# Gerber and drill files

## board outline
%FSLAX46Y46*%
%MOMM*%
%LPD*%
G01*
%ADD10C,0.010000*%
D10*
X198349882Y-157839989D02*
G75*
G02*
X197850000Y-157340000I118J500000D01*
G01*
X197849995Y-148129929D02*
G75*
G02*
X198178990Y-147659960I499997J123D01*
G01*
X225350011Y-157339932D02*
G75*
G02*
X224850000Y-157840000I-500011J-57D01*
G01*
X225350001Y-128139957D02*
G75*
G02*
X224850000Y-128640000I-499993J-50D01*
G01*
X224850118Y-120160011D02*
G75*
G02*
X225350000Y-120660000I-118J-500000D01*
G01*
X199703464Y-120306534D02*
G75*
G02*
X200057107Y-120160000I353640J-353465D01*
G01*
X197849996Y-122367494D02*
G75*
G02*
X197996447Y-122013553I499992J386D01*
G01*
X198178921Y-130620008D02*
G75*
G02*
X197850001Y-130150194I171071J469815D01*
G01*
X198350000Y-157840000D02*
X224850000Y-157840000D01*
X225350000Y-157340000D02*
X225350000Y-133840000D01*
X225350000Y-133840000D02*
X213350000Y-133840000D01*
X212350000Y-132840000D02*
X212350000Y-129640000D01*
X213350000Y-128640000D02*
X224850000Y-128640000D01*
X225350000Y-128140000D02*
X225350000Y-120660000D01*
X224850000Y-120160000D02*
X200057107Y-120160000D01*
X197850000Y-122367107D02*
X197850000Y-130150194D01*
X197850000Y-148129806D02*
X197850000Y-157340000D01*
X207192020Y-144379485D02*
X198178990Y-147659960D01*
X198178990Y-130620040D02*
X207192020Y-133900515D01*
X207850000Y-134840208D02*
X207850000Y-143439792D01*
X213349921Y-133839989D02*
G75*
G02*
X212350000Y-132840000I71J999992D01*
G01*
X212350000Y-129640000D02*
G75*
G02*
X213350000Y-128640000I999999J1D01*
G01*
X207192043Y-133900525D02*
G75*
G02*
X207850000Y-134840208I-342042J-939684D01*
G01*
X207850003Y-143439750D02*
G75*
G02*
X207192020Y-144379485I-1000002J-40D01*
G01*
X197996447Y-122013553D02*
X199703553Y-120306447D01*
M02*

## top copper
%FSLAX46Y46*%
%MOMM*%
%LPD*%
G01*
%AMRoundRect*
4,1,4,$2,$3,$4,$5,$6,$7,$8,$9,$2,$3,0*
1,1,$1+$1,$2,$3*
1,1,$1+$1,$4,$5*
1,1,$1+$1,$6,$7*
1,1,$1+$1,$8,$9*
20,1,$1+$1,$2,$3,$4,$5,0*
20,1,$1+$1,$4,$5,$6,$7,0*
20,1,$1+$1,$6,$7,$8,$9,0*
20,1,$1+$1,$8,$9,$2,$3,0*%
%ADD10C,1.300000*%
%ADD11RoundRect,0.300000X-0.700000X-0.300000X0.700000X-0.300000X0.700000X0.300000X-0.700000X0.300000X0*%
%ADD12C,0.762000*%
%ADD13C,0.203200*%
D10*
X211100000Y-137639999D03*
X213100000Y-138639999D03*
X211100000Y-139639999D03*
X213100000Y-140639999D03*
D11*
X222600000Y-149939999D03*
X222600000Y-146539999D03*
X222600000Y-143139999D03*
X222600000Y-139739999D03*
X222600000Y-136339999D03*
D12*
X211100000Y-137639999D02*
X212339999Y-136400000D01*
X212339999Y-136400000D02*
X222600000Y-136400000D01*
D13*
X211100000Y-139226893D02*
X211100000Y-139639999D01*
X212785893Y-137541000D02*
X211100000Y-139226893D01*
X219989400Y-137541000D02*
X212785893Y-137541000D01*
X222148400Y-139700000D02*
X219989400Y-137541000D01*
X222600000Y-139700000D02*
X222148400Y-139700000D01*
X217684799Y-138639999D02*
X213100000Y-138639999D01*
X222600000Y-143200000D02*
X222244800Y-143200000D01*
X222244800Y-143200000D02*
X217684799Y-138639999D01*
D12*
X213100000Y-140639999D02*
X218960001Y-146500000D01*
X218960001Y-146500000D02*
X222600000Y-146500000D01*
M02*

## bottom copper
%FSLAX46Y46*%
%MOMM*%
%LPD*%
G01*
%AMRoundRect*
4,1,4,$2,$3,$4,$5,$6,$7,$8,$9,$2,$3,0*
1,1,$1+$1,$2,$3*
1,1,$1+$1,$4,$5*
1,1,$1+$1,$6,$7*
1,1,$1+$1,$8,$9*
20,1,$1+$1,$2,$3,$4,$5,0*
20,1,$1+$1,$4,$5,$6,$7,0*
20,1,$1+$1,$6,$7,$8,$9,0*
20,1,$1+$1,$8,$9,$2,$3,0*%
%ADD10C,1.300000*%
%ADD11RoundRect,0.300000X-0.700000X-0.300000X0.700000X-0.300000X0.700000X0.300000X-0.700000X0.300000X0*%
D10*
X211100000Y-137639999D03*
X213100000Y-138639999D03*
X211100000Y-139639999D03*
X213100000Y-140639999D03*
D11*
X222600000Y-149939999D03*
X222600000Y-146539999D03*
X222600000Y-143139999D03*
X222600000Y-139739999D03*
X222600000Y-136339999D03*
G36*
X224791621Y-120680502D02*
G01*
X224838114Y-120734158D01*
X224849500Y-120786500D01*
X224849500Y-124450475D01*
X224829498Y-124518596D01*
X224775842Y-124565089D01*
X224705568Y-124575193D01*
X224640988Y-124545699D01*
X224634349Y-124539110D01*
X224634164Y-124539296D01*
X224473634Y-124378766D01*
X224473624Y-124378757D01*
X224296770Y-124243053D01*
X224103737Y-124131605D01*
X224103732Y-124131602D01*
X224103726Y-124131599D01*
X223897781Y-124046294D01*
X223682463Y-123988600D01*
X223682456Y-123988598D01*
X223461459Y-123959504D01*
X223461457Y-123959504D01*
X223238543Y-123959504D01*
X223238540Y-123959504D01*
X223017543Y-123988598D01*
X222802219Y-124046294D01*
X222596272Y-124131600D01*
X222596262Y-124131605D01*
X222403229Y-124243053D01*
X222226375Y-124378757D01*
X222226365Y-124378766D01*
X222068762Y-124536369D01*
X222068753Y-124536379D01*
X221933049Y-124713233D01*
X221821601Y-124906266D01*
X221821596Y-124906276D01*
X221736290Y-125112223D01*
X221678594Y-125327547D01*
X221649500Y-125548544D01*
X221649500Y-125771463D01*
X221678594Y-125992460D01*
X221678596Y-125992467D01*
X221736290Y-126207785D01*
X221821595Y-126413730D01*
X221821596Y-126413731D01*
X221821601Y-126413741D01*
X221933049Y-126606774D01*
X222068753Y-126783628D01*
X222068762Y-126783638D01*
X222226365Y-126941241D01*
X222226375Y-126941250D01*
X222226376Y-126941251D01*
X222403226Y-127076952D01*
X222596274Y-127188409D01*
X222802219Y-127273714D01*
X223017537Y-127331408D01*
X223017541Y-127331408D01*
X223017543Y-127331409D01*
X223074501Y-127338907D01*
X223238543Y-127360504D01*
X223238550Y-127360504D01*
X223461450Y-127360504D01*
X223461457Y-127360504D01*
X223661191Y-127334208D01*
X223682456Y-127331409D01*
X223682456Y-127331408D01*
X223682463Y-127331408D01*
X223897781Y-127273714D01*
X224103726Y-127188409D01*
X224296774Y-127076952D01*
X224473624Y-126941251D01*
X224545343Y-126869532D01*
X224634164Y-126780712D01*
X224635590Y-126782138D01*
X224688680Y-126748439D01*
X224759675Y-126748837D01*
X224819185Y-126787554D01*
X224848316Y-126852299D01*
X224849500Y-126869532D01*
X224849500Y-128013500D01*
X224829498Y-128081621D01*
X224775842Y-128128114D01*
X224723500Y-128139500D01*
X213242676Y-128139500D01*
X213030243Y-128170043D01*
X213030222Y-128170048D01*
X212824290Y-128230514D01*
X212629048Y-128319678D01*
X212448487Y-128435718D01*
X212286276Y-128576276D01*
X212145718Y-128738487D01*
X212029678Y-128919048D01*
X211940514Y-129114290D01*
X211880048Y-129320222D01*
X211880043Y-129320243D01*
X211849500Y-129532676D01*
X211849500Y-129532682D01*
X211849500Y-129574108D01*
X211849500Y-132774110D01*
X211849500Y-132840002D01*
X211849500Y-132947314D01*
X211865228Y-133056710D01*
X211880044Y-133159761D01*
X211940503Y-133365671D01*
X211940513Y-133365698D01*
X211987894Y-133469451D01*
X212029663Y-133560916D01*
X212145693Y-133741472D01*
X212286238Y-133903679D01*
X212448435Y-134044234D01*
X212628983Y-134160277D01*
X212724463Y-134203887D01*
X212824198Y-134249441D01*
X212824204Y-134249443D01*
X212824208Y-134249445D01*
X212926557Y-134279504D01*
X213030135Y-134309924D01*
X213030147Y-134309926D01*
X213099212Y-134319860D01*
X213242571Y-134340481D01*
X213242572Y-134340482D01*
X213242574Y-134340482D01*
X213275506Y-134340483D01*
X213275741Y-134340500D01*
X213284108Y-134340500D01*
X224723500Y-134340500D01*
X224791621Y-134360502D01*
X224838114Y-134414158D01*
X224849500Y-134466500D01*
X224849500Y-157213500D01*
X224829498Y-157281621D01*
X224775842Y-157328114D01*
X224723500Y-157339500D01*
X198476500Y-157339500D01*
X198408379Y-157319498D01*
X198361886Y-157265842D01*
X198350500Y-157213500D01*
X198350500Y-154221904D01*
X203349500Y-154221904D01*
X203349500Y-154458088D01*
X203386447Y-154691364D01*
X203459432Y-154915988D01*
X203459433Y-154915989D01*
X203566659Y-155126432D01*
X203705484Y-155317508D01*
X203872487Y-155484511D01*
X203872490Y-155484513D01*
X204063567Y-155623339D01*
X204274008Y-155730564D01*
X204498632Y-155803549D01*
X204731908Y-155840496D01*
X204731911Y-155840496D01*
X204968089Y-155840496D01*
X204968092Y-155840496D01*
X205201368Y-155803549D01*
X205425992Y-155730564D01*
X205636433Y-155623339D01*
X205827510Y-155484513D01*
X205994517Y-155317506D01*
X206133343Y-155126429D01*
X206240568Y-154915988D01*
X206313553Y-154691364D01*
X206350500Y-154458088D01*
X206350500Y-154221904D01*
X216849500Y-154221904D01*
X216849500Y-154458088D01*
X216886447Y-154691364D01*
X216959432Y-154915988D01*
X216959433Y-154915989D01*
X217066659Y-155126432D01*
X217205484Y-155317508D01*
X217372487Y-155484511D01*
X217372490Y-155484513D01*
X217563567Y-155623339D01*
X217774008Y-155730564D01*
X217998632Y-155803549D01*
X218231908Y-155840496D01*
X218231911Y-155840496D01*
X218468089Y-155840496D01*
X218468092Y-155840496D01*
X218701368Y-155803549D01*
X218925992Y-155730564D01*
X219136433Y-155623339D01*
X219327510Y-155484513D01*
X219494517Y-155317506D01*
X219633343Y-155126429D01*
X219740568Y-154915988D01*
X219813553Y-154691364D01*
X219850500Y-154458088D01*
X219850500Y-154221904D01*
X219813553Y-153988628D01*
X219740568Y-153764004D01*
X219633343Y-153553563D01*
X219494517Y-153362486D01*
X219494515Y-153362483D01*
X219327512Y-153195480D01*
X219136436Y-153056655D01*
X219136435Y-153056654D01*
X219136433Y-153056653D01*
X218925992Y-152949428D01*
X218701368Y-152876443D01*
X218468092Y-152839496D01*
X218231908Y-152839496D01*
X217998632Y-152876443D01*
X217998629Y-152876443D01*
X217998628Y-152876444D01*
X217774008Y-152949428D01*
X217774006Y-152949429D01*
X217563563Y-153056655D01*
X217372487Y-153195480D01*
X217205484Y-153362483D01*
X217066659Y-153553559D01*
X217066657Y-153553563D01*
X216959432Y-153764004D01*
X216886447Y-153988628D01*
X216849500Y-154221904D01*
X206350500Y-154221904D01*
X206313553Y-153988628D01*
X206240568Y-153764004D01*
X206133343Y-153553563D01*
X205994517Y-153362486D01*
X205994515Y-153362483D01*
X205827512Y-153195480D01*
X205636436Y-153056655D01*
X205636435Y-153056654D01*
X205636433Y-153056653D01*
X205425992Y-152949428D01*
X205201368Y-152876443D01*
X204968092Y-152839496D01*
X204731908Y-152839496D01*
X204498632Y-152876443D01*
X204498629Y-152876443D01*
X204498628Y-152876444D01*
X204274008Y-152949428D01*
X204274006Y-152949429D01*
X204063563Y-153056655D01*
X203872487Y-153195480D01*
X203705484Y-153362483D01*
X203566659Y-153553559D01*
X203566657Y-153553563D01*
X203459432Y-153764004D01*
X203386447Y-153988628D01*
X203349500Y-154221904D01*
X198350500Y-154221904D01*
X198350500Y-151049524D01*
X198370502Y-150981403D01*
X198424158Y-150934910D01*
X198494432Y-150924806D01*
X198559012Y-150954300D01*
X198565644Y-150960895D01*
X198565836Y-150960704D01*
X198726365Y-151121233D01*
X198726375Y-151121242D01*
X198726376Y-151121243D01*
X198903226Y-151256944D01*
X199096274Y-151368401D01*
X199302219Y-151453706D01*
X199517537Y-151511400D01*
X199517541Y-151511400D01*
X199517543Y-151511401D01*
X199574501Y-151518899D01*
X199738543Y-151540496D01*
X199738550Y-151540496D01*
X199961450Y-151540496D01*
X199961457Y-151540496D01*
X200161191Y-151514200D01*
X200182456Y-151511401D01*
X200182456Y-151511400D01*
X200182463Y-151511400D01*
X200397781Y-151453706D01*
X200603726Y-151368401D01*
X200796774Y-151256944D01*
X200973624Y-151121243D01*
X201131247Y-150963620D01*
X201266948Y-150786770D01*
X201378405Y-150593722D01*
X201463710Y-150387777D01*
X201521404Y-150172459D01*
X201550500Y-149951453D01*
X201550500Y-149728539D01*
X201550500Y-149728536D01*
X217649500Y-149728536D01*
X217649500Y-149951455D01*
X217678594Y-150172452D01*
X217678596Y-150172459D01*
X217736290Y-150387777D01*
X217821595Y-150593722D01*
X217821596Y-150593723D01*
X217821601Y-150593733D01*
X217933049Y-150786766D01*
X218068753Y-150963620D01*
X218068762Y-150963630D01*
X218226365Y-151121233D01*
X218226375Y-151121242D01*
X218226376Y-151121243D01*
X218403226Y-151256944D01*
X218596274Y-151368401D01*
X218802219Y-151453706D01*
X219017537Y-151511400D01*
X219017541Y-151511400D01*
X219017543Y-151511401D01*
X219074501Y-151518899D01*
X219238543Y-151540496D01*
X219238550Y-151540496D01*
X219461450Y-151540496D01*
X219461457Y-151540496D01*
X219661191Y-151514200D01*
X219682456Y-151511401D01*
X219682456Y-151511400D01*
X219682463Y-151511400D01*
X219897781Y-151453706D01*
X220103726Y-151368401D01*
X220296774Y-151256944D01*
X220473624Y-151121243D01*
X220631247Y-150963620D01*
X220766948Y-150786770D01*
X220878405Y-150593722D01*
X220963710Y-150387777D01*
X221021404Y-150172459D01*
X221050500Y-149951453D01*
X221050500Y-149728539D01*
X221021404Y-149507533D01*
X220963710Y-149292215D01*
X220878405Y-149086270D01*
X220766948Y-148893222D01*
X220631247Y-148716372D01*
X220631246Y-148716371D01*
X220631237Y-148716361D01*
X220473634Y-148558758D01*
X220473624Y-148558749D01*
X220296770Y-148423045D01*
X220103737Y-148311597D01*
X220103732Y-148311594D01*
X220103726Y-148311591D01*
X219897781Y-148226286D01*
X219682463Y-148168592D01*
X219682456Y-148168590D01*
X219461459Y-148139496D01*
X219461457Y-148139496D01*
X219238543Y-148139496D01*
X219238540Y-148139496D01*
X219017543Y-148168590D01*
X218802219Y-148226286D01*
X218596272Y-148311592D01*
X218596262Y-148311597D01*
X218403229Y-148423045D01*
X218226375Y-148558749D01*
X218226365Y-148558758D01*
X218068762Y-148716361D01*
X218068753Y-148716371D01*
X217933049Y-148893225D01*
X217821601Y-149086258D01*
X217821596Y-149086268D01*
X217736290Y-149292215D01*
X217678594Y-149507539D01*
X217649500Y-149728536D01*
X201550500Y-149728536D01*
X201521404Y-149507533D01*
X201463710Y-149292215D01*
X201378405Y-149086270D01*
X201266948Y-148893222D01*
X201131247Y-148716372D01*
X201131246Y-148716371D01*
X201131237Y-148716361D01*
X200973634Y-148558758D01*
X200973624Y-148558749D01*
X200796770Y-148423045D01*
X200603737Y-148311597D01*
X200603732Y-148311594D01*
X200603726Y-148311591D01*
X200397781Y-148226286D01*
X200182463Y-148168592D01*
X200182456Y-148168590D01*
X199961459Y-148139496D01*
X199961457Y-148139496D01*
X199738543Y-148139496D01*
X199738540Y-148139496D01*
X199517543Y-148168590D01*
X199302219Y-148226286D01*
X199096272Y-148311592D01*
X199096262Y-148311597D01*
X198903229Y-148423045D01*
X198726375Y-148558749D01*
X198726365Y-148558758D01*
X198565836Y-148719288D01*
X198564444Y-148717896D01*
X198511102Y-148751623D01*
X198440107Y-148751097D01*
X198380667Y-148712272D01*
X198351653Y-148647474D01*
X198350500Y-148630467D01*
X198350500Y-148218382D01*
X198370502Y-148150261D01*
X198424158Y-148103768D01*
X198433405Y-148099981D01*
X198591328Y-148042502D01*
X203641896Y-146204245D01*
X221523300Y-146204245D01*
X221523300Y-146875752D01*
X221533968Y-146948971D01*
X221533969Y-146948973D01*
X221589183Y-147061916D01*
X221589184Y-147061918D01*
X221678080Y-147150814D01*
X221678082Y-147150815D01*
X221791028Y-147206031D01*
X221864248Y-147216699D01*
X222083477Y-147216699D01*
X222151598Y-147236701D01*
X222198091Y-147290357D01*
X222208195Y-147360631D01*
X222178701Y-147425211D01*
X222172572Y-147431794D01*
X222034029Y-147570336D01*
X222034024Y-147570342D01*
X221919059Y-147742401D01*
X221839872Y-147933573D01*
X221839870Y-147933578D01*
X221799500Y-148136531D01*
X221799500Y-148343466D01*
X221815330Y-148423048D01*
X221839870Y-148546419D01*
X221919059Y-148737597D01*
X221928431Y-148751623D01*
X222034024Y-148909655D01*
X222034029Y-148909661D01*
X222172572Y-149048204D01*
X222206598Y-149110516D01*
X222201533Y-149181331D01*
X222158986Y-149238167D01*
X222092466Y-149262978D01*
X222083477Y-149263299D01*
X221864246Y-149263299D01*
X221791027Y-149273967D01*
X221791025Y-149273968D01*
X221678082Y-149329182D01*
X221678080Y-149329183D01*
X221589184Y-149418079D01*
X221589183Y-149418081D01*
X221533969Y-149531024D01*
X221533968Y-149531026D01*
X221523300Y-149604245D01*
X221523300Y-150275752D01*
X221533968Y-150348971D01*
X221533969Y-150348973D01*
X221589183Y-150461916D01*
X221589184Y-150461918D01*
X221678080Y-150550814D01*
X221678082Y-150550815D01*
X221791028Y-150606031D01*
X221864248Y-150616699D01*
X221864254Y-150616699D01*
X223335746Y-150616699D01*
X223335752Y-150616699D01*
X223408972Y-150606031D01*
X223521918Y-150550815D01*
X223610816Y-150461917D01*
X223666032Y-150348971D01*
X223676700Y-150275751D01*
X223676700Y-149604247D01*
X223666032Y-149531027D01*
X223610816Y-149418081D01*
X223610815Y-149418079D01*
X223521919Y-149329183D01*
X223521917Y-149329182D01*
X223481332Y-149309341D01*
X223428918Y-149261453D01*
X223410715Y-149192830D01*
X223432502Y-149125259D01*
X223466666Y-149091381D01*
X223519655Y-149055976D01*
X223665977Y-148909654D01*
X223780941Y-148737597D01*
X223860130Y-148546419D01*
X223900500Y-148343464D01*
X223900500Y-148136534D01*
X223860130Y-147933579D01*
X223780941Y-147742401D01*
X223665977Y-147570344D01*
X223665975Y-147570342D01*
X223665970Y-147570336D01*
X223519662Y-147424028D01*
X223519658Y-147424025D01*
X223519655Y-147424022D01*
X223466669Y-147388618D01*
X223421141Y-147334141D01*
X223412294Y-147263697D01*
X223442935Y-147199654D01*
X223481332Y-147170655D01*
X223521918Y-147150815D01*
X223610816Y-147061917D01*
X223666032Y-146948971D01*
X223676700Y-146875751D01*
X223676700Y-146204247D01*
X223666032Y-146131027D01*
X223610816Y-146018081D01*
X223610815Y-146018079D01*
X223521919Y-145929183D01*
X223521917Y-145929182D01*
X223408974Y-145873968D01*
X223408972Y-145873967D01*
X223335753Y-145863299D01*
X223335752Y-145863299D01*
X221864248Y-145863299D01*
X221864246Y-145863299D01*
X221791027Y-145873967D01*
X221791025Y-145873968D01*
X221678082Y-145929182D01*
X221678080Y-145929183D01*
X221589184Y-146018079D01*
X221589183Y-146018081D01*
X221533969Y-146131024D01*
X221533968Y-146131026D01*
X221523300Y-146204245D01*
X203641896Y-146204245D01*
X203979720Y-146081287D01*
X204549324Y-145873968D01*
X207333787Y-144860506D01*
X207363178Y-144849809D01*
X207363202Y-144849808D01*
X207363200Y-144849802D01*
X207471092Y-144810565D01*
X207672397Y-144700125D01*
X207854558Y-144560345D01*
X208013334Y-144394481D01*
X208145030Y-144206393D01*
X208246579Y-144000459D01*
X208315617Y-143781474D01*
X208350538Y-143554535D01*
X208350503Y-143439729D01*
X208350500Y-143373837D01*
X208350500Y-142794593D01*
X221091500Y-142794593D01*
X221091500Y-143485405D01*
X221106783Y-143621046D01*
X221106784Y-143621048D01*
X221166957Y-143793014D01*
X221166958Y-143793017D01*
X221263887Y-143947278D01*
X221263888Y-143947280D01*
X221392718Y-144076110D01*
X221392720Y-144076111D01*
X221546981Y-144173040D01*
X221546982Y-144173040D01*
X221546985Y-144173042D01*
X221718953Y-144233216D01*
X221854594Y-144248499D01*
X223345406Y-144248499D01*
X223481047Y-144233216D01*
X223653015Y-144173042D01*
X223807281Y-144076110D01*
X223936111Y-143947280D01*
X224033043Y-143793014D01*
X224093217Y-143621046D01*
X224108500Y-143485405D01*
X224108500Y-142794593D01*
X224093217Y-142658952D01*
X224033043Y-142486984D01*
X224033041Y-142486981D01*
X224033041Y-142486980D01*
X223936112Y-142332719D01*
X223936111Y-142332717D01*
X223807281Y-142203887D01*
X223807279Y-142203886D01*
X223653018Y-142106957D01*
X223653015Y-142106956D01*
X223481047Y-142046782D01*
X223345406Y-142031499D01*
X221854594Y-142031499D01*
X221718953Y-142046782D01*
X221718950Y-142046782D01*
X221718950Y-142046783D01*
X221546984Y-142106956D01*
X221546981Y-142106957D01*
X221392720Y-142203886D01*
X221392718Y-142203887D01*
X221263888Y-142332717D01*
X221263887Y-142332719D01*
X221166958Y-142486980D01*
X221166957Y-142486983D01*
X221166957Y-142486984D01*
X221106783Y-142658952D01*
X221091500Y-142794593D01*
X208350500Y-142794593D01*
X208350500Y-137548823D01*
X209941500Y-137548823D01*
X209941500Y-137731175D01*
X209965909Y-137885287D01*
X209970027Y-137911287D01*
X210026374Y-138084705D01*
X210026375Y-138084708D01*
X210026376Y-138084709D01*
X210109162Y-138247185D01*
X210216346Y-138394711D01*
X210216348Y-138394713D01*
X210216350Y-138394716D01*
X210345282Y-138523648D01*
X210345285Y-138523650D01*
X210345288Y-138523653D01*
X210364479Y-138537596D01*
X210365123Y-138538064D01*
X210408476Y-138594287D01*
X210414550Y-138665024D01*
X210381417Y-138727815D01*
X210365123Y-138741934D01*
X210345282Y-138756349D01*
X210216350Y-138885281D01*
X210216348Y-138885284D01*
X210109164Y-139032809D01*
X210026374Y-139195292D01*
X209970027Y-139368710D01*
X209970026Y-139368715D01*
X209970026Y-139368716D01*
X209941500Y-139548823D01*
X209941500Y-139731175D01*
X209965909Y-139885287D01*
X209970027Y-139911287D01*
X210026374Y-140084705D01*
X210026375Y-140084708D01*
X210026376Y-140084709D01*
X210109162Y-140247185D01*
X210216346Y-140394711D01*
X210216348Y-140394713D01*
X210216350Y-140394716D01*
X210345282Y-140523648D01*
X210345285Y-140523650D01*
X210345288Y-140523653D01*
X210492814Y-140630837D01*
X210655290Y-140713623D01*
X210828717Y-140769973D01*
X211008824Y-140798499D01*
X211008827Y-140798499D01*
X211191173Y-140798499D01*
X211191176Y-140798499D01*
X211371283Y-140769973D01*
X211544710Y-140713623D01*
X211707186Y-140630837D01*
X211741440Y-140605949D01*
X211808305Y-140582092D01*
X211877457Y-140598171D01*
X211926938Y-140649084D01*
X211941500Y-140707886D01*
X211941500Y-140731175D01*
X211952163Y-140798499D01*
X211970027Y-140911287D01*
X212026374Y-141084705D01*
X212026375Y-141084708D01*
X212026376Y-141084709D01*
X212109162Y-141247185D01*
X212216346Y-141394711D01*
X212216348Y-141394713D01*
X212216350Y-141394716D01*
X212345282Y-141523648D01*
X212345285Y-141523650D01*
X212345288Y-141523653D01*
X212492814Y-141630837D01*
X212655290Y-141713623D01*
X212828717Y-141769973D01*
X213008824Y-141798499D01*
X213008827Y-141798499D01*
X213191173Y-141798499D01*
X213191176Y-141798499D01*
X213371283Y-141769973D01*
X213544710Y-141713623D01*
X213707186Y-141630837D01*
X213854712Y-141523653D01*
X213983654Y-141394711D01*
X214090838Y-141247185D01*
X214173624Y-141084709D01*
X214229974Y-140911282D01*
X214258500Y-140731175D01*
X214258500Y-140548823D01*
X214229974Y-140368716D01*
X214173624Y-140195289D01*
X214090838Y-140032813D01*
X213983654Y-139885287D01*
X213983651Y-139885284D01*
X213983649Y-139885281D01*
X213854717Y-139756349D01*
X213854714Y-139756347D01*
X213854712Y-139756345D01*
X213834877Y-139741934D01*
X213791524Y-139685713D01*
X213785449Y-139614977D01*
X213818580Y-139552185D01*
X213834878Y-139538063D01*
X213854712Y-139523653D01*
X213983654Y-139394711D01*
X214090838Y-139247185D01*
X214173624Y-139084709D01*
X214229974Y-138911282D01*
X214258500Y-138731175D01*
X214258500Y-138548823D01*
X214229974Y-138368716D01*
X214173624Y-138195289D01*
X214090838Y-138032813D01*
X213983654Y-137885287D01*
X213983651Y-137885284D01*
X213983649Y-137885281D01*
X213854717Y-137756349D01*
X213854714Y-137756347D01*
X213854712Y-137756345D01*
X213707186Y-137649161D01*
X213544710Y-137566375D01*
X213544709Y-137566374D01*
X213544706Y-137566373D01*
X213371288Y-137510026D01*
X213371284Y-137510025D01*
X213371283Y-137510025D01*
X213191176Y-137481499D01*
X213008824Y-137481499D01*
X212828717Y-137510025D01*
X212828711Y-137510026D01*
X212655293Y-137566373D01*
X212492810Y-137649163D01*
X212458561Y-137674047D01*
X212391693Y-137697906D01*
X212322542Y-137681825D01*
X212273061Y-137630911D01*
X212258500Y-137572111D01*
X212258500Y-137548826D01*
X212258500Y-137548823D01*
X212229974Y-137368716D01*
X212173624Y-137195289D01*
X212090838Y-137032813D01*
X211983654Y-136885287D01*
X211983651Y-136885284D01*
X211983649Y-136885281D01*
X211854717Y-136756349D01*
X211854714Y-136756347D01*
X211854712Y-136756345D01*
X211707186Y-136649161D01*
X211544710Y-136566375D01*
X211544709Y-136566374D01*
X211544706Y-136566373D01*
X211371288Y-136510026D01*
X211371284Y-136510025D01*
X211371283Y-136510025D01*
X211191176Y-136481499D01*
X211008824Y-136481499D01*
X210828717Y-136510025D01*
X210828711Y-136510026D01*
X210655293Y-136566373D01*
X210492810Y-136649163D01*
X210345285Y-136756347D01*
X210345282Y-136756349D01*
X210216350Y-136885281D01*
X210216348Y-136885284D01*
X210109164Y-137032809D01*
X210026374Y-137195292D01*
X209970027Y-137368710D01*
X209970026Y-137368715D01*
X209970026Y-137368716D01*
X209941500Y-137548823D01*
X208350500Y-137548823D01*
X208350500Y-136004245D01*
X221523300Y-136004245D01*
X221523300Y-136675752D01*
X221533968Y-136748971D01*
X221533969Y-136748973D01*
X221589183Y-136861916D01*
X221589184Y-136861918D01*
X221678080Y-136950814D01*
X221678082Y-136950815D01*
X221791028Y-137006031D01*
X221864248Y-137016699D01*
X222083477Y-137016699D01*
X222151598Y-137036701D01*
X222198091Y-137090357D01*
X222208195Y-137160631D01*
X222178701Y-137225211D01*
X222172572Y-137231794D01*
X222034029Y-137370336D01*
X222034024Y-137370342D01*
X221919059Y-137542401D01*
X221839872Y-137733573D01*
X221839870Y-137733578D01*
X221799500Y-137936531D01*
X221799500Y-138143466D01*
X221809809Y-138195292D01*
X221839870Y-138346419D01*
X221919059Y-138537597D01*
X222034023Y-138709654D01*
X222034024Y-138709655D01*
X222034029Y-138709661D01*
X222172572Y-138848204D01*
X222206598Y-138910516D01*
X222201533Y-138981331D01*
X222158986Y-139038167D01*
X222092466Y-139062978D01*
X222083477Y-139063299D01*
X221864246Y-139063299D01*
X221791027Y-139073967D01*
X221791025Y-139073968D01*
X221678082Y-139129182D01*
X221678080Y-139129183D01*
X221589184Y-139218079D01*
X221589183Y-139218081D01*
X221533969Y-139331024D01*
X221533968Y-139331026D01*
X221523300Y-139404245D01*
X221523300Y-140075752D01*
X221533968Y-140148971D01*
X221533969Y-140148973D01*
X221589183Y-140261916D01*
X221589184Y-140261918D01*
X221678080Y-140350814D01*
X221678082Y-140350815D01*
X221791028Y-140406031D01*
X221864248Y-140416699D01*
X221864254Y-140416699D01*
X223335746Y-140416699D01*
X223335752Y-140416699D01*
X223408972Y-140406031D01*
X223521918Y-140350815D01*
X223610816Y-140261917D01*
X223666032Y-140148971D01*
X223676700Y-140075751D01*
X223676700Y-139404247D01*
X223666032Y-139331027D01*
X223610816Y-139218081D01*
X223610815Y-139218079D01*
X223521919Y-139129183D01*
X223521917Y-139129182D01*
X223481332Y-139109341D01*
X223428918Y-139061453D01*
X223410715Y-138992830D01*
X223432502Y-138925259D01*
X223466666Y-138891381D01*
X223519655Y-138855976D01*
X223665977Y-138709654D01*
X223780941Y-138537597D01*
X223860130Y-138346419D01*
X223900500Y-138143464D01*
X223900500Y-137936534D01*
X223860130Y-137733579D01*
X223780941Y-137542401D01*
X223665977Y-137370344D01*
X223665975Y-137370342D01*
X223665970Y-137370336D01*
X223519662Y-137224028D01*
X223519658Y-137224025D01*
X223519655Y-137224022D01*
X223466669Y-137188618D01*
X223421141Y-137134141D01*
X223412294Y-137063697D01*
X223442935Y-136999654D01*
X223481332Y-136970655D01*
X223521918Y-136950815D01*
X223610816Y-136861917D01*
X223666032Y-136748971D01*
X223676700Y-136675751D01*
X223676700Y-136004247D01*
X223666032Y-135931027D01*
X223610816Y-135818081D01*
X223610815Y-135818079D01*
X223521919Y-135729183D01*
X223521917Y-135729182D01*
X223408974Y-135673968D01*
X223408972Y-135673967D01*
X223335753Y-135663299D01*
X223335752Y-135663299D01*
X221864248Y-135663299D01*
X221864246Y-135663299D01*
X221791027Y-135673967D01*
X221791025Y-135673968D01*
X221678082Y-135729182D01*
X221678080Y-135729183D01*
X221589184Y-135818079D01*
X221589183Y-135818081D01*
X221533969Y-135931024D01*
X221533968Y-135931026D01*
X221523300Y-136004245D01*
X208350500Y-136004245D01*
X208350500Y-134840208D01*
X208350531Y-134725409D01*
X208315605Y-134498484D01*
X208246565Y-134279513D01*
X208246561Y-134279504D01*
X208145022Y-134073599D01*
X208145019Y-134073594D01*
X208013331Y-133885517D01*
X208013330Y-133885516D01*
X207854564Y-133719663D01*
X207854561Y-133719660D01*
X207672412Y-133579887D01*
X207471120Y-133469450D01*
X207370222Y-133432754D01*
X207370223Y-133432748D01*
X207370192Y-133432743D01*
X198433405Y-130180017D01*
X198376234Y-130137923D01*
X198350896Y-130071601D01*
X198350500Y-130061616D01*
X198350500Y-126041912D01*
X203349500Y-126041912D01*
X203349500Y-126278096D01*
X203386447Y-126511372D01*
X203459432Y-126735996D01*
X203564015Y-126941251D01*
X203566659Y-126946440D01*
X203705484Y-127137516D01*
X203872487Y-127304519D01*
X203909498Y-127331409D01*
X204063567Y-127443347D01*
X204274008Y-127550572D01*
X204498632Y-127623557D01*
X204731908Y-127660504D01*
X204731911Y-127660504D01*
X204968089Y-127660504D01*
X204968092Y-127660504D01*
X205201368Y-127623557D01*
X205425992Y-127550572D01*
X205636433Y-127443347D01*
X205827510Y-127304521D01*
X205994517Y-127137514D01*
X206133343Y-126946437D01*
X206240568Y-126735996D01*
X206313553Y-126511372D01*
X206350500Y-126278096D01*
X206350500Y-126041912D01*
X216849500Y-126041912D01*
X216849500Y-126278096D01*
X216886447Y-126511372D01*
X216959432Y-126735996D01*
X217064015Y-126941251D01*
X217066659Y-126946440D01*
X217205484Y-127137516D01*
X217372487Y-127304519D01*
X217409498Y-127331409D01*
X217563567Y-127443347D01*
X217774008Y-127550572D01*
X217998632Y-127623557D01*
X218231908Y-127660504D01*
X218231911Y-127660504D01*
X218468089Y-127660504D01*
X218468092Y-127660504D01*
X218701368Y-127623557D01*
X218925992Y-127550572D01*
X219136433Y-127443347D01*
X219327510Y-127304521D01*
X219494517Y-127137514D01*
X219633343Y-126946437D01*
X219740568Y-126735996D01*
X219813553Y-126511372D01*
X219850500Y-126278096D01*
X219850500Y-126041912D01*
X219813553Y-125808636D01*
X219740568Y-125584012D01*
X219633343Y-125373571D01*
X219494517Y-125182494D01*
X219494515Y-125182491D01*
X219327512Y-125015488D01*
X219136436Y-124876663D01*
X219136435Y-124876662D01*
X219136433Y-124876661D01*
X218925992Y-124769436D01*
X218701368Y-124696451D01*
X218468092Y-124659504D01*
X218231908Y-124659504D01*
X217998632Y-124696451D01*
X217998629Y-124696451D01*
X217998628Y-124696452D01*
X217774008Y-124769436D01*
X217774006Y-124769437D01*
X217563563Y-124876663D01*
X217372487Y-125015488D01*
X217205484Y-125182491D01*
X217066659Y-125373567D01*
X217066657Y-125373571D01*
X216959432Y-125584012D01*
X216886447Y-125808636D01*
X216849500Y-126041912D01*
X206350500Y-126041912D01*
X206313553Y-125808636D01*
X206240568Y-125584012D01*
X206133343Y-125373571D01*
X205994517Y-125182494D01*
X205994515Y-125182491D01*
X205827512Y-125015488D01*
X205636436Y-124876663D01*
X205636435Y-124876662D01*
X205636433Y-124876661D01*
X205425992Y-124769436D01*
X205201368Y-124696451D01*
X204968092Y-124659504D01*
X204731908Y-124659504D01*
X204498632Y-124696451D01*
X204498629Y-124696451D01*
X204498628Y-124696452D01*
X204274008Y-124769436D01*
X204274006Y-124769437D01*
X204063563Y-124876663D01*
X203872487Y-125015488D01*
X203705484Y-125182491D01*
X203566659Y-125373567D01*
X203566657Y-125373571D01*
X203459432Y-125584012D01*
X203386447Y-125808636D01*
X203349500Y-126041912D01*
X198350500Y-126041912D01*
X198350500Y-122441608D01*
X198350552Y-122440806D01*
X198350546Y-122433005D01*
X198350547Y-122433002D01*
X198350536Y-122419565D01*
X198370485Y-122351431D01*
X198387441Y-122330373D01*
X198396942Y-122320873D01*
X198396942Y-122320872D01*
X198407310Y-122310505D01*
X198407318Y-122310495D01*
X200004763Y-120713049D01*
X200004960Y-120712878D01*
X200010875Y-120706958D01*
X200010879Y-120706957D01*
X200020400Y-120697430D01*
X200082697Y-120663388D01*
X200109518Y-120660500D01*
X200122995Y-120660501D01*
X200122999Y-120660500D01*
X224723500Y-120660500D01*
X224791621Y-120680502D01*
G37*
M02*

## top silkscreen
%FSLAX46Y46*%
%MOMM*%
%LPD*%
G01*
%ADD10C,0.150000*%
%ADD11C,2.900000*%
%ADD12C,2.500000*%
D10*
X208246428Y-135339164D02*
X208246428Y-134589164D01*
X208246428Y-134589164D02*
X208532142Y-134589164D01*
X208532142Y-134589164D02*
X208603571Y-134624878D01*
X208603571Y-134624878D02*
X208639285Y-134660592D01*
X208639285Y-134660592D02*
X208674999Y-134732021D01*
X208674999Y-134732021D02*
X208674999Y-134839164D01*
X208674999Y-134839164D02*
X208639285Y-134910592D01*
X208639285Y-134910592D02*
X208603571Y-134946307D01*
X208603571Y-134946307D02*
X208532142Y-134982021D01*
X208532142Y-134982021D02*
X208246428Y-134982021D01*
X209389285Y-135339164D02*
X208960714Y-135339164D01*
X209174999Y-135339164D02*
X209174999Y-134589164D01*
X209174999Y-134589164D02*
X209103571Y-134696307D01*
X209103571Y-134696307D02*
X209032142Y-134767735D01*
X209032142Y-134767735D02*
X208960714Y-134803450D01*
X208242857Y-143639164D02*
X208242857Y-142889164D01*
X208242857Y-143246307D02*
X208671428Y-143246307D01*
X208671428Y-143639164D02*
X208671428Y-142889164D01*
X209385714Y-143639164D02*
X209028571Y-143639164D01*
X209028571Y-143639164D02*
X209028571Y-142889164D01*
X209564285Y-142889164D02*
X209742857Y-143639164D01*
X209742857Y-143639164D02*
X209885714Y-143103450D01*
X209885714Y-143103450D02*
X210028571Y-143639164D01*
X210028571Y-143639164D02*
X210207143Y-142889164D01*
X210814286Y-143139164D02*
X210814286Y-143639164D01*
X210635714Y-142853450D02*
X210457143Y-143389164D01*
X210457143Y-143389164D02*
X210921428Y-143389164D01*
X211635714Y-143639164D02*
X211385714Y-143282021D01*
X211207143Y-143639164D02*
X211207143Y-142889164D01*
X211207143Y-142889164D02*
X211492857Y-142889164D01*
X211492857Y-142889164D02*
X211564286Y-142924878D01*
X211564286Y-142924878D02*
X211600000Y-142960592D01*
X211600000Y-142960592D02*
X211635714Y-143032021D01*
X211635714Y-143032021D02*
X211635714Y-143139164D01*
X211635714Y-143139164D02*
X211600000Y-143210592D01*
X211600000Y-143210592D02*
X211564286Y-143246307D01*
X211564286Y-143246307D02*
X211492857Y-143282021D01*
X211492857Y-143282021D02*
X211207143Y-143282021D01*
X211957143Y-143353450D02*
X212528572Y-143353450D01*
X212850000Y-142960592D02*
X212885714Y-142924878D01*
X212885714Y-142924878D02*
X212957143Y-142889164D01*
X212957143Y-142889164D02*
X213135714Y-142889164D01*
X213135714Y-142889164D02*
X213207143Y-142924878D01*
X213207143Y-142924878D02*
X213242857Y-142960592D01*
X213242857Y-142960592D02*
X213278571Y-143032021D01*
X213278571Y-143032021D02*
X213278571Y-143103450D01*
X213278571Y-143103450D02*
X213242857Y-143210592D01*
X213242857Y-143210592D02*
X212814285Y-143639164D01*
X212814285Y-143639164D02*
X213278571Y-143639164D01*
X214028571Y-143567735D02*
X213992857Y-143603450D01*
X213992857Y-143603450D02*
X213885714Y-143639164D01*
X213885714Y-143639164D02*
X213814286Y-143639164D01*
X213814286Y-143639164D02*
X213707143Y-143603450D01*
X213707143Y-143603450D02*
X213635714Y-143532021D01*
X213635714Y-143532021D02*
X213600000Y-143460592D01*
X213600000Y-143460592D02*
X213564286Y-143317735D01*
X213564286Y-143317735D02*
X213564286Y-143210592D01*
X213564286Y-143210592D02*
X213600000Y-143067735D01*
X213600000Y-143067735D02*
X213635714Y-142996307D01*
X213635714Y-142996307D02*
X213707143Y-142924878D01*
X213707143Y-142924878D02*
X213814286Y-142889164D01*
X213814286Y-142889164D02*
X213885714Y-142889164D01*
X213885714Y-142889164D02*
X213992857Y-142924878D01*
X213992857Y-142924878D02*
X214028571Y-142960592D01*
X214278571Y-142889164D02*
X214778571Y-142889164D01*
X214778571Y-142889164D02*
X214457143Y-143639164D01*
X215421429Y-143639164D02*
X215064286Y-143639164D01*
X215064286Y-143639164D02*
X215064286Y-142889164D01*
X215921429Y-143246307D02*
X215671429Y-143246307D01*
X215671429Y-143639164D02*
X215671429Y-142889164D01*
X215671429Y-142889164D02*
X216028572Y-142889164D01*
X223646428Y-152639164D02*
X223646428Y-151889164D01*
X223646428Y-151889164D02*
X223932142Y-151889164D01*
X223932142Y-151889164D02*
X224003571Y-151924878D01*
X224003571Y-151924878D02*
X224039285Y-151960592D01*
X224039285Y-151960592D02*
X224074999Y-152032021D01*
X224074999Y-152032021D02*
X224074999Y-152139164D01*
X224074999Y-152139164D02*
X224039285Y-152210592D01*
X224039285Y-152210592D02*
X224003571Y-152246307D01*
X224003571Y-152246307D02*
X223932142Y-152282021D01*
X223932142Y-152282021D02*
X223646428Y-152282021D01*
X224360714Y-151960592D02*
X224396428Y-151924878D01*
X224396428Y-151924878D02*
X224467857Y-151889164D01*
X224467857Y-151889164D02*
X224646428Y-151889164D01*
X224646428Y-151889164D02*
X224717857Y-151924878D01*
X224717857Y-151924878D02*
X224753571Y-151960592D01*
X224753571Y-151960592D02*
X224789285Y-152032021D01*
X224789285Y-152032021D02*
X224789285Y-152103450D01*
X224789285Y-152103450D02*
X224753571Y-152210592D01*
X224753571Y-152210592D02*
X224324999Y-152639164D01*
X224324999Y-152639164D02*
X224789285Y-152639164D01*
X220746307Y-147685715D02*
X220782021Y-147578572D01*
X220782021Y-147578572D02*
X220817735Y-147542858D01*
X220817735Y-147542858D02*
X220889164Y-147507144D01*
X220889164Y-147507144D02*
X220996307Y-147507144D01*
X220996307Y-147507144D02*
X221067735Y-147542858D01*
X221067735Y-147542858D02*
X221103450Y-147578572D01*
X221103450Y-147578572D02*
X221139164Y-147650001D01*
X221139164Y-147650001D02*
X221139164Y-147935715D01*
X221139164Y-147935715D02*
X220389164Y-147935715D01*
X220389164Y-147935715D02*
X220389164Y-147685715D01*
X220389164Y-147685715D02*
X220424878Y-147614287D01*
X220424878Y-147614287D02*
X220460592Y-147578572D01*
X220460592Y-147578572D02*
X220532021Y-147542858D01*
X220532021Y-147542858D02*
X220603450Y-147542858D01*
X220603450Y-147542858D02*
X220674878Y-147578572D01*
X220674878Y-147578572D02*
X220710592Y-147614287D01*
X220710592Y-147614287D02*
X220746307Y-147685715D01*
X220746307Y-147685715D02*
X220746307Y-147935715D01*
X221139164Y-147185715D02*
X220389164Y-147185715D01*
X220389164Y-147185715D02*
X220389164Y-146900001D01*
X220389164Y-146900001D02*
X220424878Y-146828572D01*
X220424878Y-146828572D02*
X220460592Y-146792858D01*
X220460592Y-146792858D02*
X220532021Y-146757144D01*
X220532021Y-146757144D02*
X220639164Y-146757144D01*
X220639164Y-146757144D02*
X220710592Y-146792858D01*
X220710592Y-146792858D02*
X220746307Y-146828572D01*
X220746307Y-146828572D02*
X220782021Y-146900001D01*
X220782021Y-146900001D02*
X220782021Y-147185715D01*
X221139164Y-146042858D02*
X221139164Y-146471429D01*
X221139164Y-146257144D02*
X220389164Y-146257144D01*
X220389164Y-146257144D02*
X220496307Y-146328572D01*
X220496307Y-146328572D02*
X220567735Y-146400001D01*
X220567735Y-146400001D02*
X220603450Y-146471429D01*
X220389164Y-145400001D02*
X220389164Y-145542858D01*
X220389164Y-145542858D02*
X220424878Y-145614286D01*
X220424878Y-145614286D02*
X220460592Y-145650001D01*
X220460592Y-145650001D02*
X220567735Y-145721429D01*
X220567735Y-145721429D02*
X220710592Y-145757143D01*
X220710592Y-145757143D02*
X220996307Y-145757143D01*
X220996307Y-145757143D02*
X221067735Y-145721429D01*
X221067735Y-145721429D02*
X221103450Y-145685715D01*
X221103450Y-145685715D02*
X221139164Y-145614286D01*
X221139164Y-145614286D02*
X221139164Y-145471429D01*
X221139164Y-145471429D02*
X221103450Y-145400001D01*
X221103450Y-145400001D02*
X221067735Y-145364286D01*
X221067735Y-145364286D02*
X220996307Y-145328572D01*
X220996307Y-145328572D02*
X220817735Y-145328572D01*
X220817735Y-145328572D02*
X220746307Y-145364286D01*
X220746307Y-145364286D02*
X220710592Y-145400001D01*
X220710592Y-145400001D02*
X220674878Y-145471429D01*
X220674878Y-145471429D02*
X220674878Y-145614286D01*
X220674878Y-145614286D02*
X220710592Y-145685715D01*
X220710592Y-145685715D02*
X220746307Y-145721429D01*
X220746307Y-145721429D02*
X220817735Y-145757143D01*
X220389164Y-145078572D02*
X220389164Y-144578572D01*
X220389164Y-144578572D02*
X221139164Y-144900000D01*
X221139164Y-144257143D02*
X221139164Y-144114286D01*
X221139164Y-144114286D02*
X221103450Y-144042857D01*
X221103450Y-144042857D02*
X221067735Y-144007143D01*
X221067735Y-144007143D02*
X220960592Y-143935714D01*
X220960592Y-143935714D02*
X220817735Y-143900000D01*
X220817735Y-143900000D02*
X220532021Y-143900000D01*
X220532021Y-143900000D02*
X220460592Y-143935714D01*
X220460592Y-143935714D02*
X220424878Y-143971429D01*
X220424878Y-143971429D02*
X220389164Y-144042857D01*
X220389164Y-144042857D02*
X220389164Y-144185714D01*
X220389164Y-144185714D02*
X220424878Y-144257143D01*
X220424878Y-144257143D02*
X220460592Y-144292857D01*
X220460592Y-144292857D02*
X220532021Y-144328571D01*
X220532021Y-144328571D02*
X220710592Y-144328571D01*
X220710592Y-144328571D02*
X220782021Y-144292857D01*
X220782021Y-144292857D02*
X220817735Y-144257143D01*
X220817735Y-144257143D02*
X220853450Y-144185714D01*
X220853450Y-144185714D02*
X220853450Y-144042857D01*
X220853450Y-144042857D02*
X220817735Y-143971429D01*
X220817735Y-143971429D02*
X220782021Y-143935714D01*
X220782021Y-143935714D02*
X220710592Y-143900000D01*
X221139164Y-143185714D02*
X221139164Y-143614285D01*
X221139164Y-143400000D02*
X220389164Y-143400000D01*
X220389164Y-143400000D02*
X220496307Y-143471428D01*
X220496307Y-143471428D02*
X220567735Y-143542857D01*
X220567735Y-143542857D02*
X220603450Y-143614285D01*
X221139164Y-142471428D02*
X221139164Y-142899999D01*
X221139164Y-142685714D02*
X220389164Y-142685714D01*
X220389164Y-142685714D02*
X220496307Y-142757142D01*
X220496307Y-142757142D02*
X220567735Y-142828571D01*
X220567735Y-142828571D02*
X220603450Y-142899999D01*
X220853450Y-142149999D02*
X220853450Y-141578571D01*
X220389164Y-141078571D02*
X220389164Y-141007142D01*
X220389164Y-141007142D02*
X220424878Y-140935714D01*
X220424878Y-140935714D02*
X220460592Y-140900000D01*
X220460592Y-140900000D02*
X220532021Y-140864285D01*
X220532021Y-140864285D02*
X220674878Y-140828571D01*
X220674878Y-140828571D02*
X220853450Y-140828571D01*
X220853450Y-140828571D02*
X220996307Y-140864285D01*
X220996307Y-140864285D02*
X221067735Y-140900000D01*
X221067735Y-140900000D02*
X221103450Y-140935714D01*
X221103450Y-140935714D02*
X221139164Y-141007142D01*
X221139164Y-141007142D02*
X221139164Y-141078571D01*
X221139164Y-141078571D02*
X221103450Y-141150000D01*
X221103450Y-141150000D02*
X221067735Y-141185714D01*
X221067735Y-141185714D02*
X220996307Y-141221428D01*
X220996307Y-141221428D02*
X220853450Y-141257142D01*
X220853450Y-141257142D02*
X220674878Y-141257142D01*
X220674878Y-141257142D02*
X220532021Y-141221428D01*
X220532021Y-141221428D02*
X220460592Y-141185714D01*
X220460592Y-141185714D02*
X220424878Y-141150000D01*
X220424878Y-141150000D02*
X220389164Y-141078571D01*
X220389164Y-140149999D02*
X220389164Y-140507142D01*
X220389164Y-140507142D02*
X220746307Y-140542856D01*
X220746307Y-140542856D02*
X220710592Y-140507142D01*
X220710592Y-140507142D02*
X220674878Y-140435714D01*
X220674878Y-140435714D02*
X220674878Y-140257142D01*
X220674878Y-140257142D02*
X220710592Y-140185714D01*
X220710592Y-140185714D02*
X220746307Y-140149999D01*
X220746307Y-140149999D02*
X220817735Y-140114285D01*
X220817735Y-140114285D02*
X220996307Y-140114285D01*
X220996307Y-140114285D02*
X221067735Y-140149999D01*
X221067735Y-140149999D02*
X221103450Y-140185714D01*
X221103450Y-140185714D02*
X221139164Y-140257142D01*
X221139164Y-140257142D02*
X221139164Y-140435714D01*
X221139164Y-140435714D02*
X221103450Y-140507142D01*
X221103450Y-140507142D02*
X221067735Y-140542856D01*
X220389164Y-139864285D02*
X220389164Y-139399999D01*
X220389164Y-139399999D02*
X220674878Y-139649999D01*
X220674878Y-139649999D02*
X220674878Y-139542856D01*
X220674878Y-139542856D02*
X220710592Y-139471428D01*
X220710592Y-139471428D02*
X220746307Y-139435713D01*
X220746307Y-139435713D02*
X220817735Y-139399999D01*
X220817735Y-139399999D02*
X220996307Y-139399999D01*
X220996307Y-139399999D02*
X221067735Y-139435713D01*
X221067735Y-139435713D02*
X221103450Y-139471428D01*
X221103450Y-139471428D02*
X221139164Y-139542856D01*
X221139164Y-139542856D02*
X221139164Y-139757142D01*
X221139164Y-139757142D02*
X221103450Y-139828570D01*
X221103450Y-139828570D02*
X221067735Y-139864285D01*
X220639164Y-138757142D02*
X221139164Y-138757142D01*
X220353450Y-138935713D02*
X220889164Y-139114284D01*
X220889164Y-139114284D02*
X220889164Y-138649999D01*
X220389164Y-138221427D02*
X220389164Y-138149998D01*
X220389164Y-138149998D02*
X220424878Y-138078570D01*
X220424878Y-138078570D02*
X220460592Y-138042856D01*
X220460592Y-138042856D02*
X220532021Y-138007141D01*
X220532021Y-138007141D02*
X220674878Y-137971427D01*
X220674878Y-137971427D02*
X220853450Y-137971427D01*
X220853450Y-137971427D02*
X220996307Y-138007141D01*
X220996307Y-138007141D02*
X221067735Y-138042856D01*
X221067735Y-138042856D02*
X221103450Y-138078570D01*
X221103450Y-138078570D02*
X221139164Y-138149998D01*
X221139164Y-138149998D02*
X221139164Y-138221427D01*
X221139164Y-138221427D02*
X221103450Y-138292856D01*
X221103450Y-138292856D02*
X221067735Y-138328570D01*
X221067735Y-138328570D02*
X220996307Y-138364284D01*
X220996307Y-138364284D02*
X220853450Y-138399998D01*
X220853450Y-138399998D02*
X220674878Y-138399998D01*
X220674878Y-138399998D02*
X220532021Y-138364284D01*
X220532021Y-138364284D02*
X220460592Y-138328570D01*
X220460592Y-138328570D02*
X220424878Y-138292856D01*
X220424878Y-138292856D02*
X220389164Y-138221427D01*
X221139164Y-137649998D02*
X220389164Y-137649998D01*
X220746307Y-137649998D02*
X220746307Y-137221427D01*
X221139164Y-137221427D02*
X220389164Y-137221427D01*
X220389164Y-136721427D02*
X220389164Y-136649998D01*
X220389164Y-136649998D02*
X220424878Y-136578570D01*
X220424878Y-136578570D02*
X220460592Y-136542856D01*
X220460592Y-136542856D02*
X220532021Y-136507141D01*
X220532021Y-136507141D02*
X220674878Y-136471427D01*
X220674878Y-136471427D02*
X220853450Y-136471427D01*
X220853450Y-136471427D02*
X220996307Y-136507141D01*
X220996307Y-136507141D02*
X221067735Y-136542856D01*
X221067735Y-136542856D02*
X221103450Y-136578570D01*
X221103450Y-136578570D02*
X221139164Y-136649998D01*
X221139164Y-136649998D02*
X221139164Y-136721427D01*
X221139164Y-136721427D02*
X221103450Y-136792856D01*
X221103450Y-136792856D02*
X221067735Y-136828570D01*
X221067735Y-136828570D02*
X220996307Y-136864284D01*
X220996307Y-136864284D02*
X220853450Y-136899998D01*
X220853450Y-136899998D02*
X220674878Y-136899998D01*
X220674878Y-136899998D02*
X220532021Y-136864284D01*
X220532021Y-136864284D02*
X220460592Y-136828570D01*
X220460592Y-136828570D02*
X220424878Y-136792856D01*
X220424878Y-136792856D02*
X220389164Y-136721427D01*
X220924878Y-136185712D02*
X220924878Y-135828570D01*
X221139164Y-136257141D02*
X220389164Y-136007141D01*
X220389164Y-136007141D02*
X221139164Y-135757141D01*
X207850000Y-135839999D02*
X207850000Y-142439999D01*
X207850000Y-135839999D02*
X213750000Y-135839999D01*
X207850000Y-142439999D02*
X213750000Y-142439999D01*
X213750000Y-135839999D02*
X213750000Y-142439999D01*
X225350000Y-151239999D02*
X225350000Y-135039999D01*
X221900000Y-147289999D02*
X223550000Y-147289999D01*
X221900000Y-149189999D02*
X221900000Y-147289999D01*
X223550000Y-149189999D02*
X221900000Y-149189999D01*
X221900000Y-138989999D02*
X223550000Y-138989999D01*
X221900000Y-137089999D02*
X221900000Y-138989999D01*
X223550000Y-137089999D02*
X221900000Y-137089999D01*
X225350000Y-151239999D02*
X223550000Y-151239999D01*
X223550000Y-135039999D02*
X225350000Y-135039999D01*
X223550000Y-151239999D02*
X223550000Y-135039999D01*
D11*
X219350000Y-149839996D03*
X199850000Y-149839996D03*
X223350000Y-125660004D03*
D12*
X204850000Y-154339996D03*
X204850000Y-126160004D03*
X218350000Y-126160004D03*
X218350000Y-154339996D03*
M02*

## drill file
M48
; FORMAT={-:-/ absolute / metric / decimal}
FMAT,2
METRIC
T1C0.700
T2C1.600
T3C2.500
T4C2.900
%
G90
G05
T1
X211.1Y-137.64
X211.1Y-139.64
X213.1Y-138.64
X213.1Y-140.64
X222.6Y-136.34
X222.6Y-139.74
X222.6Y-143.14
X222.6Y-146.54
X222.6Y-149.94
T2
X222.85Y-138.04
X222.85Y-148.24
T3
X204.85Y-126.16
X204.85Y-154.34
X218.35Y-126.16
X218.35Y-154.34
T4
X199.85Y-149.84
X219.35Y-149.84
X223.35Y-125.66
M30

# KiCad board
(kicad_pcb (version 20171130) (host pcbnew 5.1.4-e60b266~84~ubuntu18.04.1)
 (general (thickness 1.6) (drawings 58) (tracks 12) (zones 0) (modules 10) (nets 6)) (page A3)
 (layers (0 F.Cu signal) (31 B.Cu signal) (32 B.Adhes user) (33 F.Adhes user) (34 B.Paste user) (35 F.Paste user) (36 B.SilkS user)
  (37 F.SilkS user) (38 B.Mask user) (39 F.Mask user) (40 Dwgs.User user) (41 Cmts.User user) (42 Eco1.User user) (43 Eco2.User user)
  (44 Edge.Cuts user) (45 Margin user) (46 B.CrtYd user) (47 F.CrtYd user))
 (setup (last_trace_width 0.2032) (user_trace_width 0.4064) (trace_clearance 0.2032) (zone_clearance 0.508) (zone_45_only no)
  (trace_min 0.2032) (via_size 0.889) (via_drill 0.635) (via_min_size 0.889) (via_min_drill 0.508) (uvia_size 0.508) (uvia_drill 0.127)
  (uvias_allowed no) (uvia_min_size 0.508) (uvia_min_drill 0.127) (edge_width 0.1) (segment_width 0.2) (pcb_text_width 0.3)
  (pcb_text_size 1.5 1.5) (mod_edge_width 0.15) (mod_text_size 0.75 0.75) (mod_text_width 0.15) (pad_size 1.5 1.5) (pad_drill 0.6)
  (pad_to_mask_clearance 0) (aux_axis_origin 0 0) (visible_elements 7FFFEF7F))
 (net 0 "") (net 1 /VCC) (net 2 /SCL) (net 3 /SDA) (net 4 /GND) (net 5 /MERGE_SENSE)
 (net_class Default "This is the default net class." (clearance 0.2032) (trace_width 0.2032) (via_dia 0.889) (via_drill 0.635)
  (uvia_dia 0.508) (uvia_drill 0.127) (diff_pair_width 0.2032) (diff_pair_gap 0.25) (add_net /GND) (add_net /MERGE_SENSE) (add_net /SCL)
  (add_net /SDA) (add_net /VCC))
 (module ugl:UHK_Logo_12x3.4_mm (layer B.Cu) (at 209.8 149.8 180)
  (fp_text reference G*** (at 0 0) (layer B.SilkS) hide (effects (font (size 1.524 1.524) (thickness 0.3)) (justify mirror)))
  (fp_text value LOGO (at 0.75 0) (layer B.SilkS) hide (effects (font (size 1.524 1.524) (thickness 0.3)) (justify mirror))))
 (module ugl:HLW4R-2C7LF (layer F.Cu) (at 207.85 139.139999 270)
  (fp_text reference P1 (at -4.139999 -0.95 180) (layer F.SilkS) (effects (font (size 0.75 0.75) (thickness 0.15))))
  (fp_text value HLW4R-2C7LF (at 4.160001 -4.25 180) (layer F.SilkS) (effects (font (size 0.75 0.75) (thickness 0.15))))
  (fp_line (start -3.3 0) (end 3.3 0) (layer F.SilkS) (width 0.15))
  (fp_line (start -3.3 0) (end -3.3 -5.9) (layer F.SilkS) (width 0.15))
  (fp_line (start 3.3 0) (end 3.3 -5.9) (layer F.SilkS) (width 0.15))
  (fp_line (start -3.3 -5.9) (end 3.3 -5.9) (layer F.SilkS) (width 0.15))
  (pad 4 thru_hole circle (at -1.5 -3.25 270) (size 1.3 1.3) (drill 0.7) (layers *.Cu *.Mask) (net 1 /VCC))
  (pad 3 thru_hole circle (at -0.5 -5.25 270) (size 1.3 1.3) (drill 0.7) (layers *.Cu *.Mask) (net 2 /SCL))
  (pad 2 thru_hole circle (at 0.5 -3.25 270) (size 1.3 1.3) (drill 0.7) (layers *.Cu *.Mask) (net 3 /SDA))
  (pad 1 thru_hole circle (at 1.5 -5.25 270) (size 1.3 1.3) (drill 0.7) (layers *.Cu *.Mask) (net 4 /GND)))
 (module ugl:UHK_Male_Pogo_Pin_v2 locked (layer F.Cu) (at 225.35 143.139999)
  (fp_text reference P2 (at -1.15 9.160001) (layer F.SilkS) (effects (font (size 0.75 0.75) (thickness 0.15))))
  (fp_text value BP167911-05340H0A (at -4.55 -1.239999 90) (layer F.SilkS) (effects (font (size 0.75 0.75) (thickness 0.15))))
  (fp_line (start 0 8.1) (end 0 -8.1) (layer F.SilkS) (width 0.15))
  (fp_line (start -3.45 4.15) (end -1.8 4.15) (layer F.SilkS) (width 0.15))
  (fp_line (start -3.45 6.05) (end -3.45 4.15) (layer F.SilkS) (width 0.15))
  (fp_line (start -1.8 6.05) (end -3.45 6.05) (layer F.SilkS) (width 0.15))
  (fp_line (start -3.45 -4.15) (end -1.8 -4.15) (layer F.SilkS) (width 0.15))
  (fp_line (start -3.45 -6.05) (end -3.45 -4.15) (layer F.SilkS) (width 0.15))
  (fp_line (start -1.8 -6.05) (end -3.45 -6.05) (layer F.SilkS) (width 0.15))
  (fp_line (start 0 8.1) (end -1.8 8.1) (layer F.SilkS) (width 0.15))
  (fp_line (start -1.8 -8.1) (end 0 -8.1) (layer F.SilkS) (width 0.15))
  (fp_line (start -1.8 8.1) (end -1.8 -8.1) (layer F.SilkS) (width 0.15))
  (pad "" np_thru_hole circle (at -2.5 5.1 180) (size 1.6 1.6) (drill 1.6) (layers *.Cu *.Mask) (clearance 0.00254))
  (pad "" np_thru_hole circle (at -2.5 -5.1) (size 1.6 1.6) (drill 1.6) (layers *.Cu *.Mask) (clearance 0.00254))
  (pad 5 thru_hole roundrect (at -2.75 6.8) (size 2 1.2) (drill 0.7) (layers *.Cu *.Mask) (roundrect_rratio 0.25) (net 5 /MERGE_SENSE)
   (clearance 0.0762))
  (pad 4 thru_hole roundrect (at -2.75 3.4) (size 2 1.2) (drill 0.7) (layers *.Cu *.Mask) (roundrect_rratio 0.25) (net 4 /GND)
   (clearance 0.0762))
  (pad 3 thru_hole roundrect (at -2.75 0) (size 2 1.2) (drill 0.7) (layers *.Cu *.Mask) (roundrect_rratio 0.25) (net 2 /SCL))
  (pad 2 thru_hole roundrect (at -2.75 -3.4) (size 2 1.2) (drill 0.7) (layers *.Cu *.Mask) (roundrect_rratio 0.25) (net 3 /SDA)
   (clearance 0.0762))
  (pad 1 thru_hole roundrect (at -2.75 -6.8) (size 2 1.2) (drill 0.7) (layers *.Cu *.Mask) (roundrect_rratio 0.25) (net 1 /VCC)
   (clearance 0.0762)))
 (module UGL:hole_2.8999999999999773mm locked (layer F.Cu) (at 219.35 149.839996)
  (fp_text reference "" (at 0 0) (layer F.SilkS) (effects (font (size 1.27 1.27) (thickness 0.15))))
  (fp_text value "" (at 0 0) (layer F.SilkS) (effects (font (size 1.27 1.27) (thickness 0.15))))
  (pad "" np_thru_hole circle (at 0 0) (size 2.9 2.9) (drill 2.9) (layers *.Cu *.Mask F.SilkS) (clearance 0.00001)))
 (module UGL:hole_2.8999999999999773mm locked (layer F.Cu) (at 199.85 149.839996)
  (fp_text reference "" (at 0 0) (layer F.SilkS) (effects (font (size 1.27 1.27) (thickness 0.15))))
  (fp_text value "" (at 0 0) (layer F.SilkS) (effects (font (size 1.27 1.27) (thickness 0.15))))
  (pad "" np_thru_hole circle (at 0 0) (size 2.9 2.9) (drill 2.9) (layers *.Cu *.Mask F.SilkS) (clearance 0.00001)))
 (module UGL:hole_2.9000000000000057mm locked (layer F.Cu) (at 223.35 125.660004)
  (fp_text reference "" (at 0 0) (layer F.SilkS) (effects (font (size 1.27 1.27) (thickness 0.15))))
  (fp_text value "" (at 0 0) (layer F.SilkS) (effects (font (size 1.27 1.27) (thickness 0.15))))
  (pad "" np_thru_hole circle (at 0 0) (size 2.9 2.9) (drill 2.9) (layers *.Cu *.Mask F.SilkS) (clearance 0.00001)))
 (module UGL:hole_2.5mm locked (layer F.Cu) (at 204.85 154.339996)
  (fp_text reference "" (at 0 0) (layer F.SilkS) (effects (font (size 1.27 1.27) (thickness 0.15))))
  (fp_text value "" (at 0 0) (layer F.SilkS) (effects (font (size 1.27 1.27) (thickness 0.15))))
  (pad "" np_thru_hole circle (at 0 0) (size 2.5 2.5) (drill 2.5) (layers *.Cu *.Mask F.SilkS) (clearance 0.00001)))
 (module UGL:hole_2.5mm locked (layer F.Cu) (at 204.85 126.160004)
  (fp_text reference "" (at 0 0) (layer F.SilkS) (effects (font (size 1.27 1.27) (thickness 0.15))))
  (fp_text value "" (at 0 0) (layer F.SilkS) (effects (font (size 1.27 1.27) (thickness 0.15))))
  (pad "" np_thru_hole circle (at 0 0) (size 2.5 2.5) (drill 2.5) (layers *.Cu *.Mask F.SilkS) (clearance 0.00001)))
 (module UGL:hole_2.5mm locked (layer F.Cu) (at 218.35 126.160004)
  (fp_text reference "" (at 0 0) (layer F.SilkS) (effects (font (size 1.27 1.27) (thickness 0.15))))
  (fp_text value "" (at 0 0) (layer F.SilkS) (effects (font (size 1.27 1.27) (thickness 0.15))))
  (pad "" np_thru_hole circle (at 0 0) (size 2.5 2.5) (drill 2.5) (layers *.Cu *.Mask F.SilkS) (clearance 0.00001)))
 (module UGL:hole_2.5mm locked (layer F.Cu) (at 218.35 154.339996)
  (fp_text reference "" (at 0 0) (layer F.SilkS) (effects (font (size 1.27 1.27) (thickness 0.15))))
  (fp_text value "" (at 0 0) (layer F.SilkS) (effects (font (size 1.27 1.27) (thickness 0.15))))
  (pad "" np_thru_hole circle (at 0 0) (size 2.5 2.5) (drill 2.5) (layers *.Cu *.Mask F.SilkS) (clearance 0.00001)))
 (gr_arc (start 198.35 157.339989) (end 197.85 157.34) (angle -89.98521397) (layer Edge.Cuts) (width 0.01))
 (gr_arc (start 198.349992 148.129806) (end 198.17899 147.65996) (angle -70.01492042) (layer Edge.Cuts) (width 0.01))
 (gr_arc (start 224.85 157.339989) (end 224.85 157.84) (angle -90.00654586) (layer Edge.Cuts) (width 0.01))
 (gr_arc (start 224.850008 128.140007) (end 224.85 128.64) (angle -90.00660585) (layer Edge.Cuts) (width 0.01))
 (gr_arc (start 224.85 120.660011) (end 225.35 120.66) (angle -89.98521397) (layer Edge.Cuts) (width 0.01))
 (gr_arc (start 200.057104 120.659999) (end 200.057107 120.16) (angle -45.01451802) (layer Edge.Cuts) (width 0.01))
 (gr_arc (start 198.349988 122.367108) (end 197.996447 122.013553) (angle -45.04535319) (layer Edge.Cuts) (width 0.01))
 (gr_arc (start 198.349992 130.150193) (end 197.85 130.150194) (angle -69.99208089) (layer Edge.Cuts) (width 0.01))
 (gr_line (start 198.35 157.84) (end 224.85 157.84) (angle 90) (layer Edge.Cuts) (width 0.01))
 (gr_line (start 225.35 157.34) (end 225.35 133.84) (angle 90) (layer Edge.Cuts) (width 0.01))
 (gr_line (start 225.35 133.84) (end 213.35 133.84) (angle 90) (layer Edge.Cuts) (width 0.01))
 (gr_line (start 212.35 132.84) (end 212.35 129.64) (angle 90) (layer Edge.Cuts) (width 0.01))
 (gr_line (start 213.35 128.64) (end 224.85 128.64) (angle 90) (layer Edge.Cuts) (width 0.01))
 (gr_line (start 225.35 128.14) (end 225.35 120.66) (angle 90) (layer Edge.Cuts) (width 0.01))
 (gr_line (start 224.85 120.16) (end 200.057107 120.16) (angle 90) (layer Edge.Cuts) (width 0.01))
 (gr_line (start 197.85 122.367107) (end 197.85 130.150194) (angle 90) (layer Edge.Cuts) (width 0.01))
 (gr_line (start 197.85 148.129806) (end 197.85 157.34) (angle 90) (layer Edge.Cuts) (width 0.01))
 (gr_line (start 207.19202 144.379485) (end 198.17899 147.65996) (angle 90) (layer Edge.Cuts) (width 0.01))
 (gr_line (start 198.17899 130.62004) (end 207.19202 133.900515) (angle 90) (layer Edge.Cuts) (width 0.01))
 (gr_line (start 207.85 134.840208) (end 207.85 143.439792) (angle 90) (layer Edge.Cuts) (width 0.01))
 (gr_arc (start 213.349992 132.839997) (end 212.35 132.84) (angle -89.99574177) (layer Edge.Cuts) (width 0.01))
 (gr_arc (start 213.349999 129.639999) (end 213.35 128.64) (angle -90.00012957) (layer Edge.Cuts) (width 0.01))
 (gr_arc (start 206.850001 134.840209) (end 207.85 134.840208) (angle -69.99858612) (layer Edge.Cuts) (width 0.01))
 (gr_arc (start 206.850001 143.43979) (end 207.19202 144.379485) (angle -70.00237317) (layer Edge.Cuts) (width 0.01))
 (gr_line (start 197.996447 122.013553) (end 199.703553 120.306447) (angle 90) (layer Edge.Cuts) (width 0.01))
 (segment (start 211.1 137.639999) (end 212.339999 136.4) (width 0.762) (layer F.Cu) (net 1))
 (segment (start 212.339999 136.4) (end 222.6 136.4) (width 0.762) (layer F.Cu) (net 1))
 (segment (start 211.1 139.226893) (end 211.1 139.639999) (width 0.2032) (layer F.Cu) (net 3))
 (segment (start 212.785893 137.541) (end 211.1 139.226893) (width 0.2032) (layer F.Cu) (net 3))
 (segment (start 219.9894 137.541) (end 212.785893 137.541) (width 0.2032) (layer F.Cu) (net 3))
 (segment (start 222.1484 139.7) (end 219.9894 137.541) (width 0.2032) (layer F.Cu) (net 3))
 (segment (start 222.6 139.7) (end 222.1484 139.7) (width 0.2032) (layer F.Cu) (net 3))
 (segment (start 217.684799 138.639999) (end 213.1 138.639999) (width 0.2032) (layer F.Cu) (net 2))
 (segment (start 222.6 143.2) (end 222.2448 143.2) (width 0.2032) (layer F.Cu) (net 2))
 (segment (start 222.2448 143.2) (end 217.684799 138.639999) (width 0.2032) (layer F.Cu) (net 2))
 (segment (start 213.1 140.639999) (end 218.960001 146.5) (width 0.762) (layer F.Cu) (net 4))
 (segment (start 218.960001 146.5) (end 222.6 146.5) (width 0.762) (layer F.Cu) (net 4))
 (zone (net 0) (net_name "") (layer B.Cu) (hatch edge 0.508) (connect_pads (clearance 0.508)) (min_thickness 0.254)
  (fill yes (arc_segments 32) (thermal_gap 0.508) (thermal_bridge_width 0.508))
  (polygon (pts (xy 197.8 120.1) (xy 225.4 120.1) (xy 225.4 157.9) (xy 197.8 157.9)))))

